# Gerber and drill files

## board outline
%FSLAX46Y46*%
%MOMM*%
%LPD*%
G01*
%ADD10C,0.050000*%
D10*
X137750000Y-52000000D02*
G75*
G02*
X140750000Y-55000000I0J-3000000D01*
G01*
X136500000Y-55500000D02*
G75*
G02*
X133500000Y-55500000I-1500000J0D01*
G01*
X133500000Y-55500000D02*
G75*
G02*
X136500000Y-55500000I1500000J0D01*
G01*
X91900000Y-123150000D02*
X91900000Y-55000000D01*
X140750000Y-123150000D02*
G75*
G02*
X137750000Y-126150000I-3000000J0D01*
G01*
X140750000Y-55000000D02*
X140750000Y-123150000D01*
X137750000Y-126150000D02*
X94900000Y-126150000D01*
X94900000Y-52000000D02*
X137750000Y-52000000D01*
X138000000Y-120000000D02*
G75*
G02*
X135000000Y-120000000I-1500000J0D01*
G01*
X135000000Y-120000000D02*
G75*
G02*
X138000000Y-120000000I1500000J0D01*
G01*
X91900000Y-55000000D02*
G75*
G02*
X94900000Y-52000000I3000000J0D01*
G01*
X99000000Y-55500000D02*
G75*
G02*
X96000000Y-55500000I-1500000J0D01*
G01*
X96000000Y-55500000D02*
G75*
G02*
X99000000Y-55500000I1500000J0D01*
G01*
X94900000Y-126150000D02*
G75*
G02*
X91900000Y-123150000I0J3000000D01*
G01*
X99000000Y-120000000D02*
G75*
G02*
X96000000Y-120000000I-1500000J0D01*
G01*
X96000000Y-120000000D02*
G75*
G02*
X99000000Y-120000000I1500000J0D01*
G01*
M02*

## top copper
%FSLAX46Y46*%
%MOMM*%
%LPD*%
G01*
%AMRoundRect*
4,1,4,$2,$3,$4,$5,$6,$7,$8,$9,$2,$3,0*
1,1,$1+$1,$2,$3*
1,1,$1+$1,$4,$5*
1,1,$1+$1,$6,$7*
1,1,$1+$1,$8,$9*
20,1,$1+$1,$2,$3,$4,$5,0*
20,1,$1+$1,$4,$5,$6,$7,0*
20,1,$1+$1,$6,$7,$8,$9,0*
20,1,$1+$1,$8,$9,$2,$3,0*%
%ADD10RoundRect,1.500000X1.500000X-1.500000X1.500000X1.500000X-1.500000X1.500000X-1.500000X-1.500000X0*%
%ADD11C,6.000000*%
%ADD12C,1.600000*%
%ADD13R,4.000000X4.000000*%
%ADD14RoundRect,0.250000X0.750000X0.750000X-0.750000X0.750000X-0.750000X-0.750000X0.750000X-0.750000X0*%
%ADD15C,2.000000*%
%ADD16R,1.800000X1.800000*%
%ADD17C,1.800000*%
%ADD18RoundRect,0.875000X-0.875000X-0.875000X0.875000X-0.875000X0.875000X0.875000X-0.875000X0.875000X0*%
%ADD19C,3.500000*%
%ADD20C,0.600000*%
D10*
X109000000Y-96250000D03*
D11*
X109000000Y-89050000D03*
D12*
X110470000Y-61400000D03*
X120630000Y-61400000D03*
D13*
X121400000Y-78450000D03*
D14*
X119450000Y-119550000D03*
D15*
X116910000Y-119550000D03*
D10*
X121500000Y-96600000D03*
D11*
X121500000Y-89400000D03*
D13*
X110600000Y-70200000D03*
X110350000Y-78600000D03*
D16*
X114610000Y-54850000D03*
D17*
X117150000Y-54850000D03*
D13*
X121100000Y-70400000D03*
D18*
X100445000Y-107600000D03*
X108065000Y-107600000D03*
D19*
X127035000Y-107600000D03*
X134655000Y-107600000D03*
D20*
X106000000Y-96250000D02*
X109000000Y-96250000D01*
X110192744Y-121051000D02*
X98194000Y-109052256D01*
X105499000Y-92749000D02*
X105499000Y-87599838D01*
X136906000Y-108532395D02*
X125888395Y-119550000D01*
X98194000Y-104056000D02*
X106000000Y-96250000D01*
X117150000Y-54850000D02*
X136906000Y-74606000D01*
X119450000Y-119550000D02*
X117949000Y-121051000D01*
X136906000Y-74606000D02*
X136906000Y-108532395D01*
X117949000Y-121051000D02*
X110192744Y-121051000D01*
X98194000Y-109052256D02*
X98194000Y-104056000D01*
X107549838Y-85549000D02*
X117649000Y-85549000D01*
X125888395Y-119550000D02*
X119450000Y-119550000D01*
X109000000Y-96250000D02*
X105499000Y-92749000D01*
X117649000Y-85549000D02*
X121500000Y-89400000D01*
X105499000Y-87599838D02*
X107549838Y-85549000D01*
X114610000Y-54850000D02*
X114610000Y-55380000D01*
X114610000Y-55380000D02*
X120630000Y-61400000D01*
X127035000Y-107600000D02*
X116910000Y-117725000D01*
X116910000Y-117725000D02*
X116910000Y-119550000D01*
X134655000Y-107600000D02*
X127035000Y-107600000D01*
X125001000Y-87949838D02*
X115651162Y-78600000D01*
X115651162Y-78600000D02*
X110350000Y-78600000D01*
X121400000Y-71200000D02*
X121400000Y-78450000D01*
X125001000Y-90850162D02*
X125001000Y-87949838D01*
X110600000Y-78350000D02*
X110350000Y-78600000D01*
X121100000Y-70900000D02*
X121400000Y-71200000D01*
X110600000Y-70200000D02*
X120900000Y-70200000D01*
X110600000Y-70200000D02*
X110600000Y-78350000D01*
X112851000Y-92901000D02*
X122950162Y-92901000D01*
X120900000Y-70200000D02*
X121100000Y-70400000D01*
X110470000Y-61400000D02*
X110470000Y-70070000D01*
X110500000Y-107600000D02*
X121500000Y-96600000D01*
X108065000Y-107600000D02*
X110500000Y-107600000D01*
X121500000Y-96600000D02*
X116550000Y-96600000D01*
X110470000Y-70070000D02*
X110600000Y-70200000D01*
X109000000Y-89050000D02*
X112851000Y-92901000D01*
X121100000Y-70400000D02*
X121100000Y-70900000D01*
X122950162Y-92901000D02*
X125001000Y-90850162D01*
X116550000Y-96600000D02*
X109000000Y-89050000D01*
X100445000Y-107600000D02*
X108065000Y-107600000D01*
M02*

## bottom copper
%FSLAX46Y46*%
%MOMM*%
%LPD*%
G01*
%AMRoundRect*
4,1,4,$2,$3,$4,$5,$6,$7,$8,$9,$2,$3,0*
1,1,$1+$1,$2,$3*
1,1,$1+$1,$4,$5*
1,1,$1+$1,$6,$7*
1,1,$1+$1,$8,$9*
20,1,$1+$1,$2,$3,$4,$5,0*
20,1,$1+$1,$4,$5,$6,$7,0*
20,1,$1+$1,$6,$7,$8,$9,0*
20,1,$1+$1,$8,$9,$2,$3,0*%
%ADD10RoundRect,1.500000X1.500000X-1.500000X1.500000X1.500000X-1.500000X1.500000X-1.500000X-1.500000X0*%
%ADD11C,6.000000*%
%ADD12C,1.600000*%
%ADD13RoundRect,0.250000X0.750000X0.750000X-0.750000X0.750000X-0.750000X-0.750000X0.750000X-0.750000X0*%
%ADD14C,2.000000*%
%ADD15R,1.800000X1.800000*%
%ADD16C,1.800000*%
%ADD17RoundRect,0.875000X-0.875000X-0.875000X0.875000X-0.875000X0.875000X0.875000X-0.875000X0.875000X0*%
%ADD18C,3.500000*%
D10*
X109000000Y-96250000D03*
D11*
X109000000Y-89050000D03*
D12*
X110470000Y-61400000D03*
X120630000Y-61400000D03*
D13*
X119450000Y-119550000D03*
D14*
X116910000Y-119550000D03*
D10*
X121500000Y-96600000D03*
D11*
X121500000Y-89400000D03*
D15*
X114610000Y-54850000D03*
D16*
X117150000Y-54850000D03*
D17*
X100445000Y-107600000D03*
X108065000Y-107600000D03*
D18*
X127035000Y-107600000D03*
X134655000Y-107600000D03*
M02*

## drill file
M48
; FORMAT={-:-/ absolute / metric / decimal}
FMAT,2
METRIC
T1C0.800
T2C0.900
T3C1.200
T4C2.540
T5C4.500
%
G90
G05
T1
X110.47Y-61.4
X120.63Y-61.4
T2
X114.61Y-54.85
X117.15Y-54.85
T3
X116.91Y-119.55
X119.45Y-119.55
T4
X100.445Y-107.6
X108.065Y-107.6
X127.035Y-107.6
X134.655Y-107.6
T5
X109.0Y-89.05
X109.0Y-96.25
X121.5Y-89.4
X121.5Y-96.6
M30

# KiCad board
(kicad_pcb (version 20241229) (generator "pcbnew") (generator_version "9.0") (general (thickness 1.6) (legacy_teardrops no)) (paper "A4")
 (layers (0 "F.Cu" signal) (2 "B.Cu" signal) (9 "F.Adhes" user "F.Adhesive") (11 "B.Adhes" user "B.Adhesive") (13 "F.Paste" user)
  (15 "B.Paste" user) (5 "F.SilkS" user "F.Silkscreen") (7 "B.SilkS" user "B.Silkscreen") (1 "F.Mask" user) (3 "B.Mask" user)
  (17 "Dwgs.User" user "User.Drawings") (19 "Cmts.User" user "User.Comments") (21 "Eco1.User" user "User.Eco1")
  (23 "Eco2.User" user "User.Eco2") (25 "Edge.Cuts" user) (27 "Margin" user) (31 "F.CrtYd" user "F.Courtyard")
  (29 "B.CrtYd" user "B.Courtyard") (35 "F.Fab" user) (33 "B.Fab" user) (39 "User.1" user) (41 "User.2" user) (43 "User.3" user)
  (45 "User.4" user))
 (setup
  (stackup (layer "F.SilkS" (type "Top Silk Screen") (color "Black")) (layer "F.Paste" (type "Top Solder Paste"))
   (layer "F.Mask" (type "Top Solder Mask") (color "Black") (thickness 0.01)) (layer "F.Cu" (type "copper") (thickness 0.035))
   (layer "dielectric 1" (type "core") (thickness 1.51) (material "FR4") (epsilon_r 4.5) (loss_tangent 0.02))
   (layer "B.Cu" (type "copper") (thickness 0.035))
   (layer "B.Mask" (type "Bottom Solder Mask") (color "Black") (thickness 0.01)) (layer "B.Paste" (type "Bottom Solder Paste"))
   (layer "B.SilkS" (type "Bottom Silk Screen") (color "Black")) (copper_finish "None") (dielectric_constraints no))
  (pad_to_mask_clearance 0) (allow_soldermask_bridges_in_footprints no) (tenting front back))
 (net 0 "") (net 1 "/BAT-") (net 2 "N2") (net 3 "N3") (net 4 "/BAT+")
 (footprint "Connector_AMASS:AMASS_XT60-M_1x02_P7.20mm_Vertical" (layer "F.Cu") (at 109 96.25 90)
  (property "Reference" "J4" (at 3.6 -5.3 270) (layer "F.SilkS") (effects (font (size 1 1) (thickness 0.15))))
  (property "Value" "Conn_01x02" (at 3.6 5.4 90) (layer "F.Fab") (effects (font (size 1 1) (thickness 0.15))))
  (pad "1" thru_hole roundrect (at 0 0 90) (size 6 6) (drill 4.5) (layers "*.Cu" "*.Mask") (remove_unused_layers no) (roundrect_rratio 0.25)
   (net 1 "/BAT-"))
  (pad "2" thru_hole circle (at 7.2 0 90) (size 6 6) (drill 4.5) (layers "*.Cu" "*.Mask") (remove_unused_layers no) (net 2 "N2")))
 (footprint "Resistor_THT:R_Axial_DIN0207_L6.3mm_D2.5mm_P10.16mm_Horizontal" (layer "F.Cu") (at 110.47 61.4)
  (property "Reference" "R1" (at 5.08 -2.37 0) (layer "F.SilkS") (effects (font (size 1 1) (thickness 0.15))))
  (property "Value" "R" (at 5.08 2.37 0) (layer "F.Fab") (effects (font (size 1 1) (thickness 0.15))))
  (pad "1" thru_hole circle (at 0 0) (size 1.6 1.6) (drill 0.8) (layers "*.Cu" "*.Mask") (remove_unused_layers no) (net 2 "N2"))
  (pad "2" thru_hole circle (at 10.16 0) (size 1.6 1.6) (drill 0.8) (layers "*.Cu" "*.Mask") (remove_unused_layers no) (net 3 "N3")))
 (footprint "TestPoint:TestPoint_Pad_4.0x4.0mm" (layer "F.Cu") (at 121.4 78.45)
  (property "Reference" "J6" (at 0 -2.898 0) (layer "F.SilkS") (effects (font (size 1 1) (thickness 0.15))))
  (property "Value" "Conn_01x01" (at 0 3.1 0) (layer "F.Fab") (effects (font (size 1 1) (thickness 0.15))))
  (pad "1" smd rect (at 0 0) (size 4 4) (layers "F.Cu" "F.Mask") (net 2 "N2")))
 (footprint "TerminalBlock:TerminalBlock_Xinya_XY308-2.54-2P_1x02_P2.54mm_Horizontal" (layer "F.Cu") (at 119.45 119.55 180)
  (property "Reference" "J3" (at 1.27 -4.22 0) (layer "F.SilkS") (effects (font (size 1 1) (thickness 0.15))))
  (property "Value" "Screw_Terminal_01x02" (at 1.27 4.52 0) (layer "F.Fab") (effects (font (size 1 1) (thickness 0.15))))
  (pad "1" thru_hole roundrect (at 0 0 180) (size 2 2) (drill 1.2) (layers "*.Cu" "*.Mask") (remove_unused_layers no)
   (roundrect_rratio 0.125) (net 1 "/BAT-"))
  (pad "2" thru_hole circle (at 2.54 0 180) (size 2 2) (drill 1.2) (layers "*.Cu" "*.Mask") (remove_unused_layers no) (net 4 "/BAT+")))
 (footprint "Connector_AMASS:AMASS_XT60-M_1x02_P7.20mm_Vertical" (layer "F.Cu") (at 121.5 96.6 90)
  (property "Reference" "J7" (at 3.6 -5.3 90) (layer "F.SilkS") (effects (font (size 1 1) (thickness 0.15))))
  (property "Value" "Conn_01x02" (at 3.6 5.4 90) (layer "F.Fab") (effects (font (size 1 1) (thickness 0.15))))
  (pad "1" thru_hole roundrect (at 0 0 90) (size 6 6) (drill 4.5) (layers "*.Cu" "*.Mask") (remove_unused_layers no) (roundrect_rratio 0.25)
   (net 2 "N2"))
  (pad "2" thru_hole circle (at 7.2 0 90) (size 6 6) (drill 4.5) (layers "*.Cu" "*.Mask") (remove_unused_layers no) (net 1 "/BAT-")))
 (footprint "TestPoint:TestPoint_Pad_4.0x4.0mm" (layer "F.Cu") (at 110.6 70.2)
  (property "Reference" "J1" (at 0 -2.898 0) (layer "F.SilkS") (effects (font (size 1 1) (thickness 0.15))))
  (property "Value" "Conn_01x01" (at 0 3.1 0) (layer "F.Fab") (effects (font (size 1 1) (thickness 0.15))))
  (pad "1" smd rect (at 0 0) (size 4 4) (layers "F.Cu" "F.Mask") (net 2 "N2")))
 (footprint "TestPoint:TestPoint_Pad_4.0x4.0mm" (layer "F.Cu") (at 110.35 78.6)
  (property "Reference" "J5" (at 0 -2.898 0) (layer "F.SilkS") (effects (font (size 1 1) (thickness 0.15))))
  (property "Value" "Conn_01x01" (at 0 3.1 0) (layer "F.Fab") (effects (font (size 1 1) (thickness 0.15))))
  (pad "1" smd rect (at 0 0) (size 4 4) (layers "F.Cu" "F.Mask") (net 2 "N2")))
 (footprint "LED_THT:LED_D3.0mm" (layer "F.Cu") (at 114.61 54.85)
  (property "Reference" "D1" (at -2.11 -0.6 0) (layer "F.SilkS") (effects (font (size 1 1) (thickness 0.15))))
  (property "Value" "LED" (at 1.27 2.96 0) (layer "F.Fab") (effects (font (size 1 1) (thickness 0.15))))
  (pad "1" thru_hole rect (at 0 0) (size 1.8 1.8) (drill 0.9) (layers "*.Cu" "*.Mask") (remove_unused_layers no) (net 3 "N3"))
  (pad "2" thru_hole circle (at 2.54 0) (size 1.8 1.8) (drill 0.9) (layers "*.Cu" "*.Mask") (remove_unused_layers no) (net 1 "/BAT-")))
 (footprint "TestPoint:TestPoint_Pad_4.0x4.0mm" (layer "F.Cu") (at 121.1 70.4)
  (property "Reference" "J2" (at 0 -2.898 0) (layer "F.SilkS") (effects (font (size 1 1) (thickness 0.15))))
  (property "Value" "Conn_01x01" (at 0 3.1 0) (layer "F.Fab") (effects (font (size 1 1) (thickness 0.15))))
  (pad "1" smd rect (at 0 0) (size 4 4) (layers "F.Cu" "F.Mask") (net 2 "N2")))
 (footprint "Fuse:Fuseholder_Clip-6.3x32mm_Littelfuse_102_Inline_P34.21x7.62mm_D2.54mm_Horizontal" (layer "B.Cu") (at 100.445 107.6)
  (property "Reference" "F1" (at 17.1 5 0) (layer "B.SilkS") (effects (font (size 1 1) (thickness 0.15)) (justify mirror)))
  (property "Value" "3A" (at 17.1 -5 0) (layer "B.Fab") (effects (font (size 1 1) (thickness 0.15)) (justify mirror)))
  (pad "1" thru_hole roundrect (at 0 0) (size 3.5 3.5) (drill 2.54) (layers "*.Cu" "*.Mask") (remove_unused_layers no)
   (roundrect_rratio 0.25) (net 2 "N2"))
  (pad "1" thru_hole roundrect (at 7.62 0) (size 3.5 3.5) (drill 2.54) (layers "*.Cu" "*.Mask") (remove_unused_layers no)
   (roundrect_rratio 0.25) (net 2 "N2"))
  (pad "2" thru_hole circle (at 26.59 0) (size 3.5 3.5) (drill 2.54) (layers "*.Cu" "*.Mask") (remove_unused_layers no) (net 4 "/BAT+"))
  (pad "2" thru_hole circle (at 34.21 0) (size 3.5 3.5) (drill 2.54) (layers "*.Cu" "*.Mask") (remove_unused_layers no) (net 4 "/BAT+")))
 (gr_arc (start 137.75 52) (mid 139.87132 52.87868) (end 140.75 55) (stroke (width 0.05) (type default)) (layer "Edge.Cuts"))
 (gr_circle (center 135 55.5) (end 135 54) (stroke (width 0.05) (type default)) (fill no) (layer "Edge.Cuts"))
 (gr_line (start 91.9 123.15) (end 91.9 55) (stroke (width 0.05) (type default)) (layer "Edge.Cuts"))
 (gr_arc (start 140.75 123.15) (mid 139.87132 125.27132) (end 137.75 126.15) (stroke (width 0.05) (type default)) (layer "Edge.Cuts"))
 (gr_line (start 140.75 55) (end 140.75 123.15) (stroke (width 0.05) (type default)) (layer "Edge.Cuts"))
 (gr_line (start 137.75 126.15) (end 94.9 126.15) (stroke (width 0.05) (type default)) (layer "Edge.Cuts"))
 (gr_line (start 94.9 52) (end 137.75 52) (stroke (width 0.05) (type default)) (layer "Edge.Cuts"))
 (gr_circle (center 136.5 120) (end 136.5 121.5) (stroke (width 0.05) (type default)) (fill no) (layer "Edge.Cuts"))
 (gr_arc (start 91.9 55) (mid 92.77868 52.87868) (end 94.9 52) (stroke (width 0.05) (type default)) (layer "Edge.Cuts"))
 (gr_circle (center 97.5 55.5) (end 97.5 57) (stroke (width 0.05) (type default)) (fill no) (layer "Edge.Cuts"))
 (gr_arc (start 94.9 126.15) (mid 92.77868 125.27132) (end 91.9 123.15) (stroke (width 0.05) (type default)) (layer "Edge.Cuts"))
 (gr_circle (center 97.5 120) (end 97.5 121.5) (stroke (width 0.05) (type default)) (fill no) (layer "Edge.Cuts"))
 (segment (start 106 96.25) (end 109 96.25) (width 0.6) (layer "F.Cu") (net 1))
 (segment (start 110.192744 121.051) (end 98.194 109.052256) (width 0.6) (layer "F.Cu") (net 1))
 (segment (start 105.499 92.749) (end 105.499 87.599838) (width 0.6) (layer "F.Cu") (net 1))
 (segment (start 136.906 108.532395) (end 125.888395 119.55) (width 0.6) (layer "F.Cu") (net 1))
 (segment (start 98.194 104.056) (end 106 96.25) (width 0.6) (layer "F.Cu") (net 1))
 (segment (start 117.15 54.85) (end 136.906 74.606) (width 0.6) (layer "F.Cu") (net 1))
 (segment (start 119.45 119.55) (end 117.949 121.051) (width 0.6) (layer "F.Cu") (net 1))
 (segment (start 136.906 74.606) (end 136.906 108.532395) (width 0.6) (layer "F.Cu") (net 1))
 (segment (start 117.949 121.051) (end 110.192744 121.051) (width 0.6) (layer "F.Cu") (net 1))
 (segment (start 98.194 109.052256) (end 98.194 104.056) (width 0.6) (layer "F.Cu") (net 1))
 (segment (start 107.549838 85.549) (end 117.649 85.549) (width 0.6) (layer "F.Cu") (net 1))
 (segment (start 125.888395 119.55) (end 119.45 119.55) (width 0.6) (layer "F.Cu") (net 1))
 (segment (start 109 96.25) (end 105.499 92.749) (width 0.6) (layer "F.Cu") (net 1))
 (segment (start 117.649 85.549) (end 121.5 89.4) (width 0.6) (layer "F.Cu") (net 1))
 (segment (start 105.499 87.599838) (end 107.549838 85.549) (width 0.6) (layer "F.Cu") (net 1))
 (segment (start 114.61 54.85) (end 114.61 55.38) (width 0.6) (layer "F.Cu") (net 3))
 (segment (start 114.61 55.38) (end 120.63 61.4) (width 0.6) (layer "F.Cu") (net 3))
 (segment (start 127.035 107.6) (end 116.91 117.725) (width 0.6) (layer "F.Cu") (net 4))
 (segment (start 116.91 117.725) (end 116.91 119.55) (width 0.6) (layer "F.Cu") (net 4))
 (segment (start 134.655 107.6) (end 127.035 107.6) (width 0.6) (layer "F.Cu") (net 4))
 (segment (start 125.001 87.949838) (end 115.651162 78.6) (width 0.6) (layer "F.Cu") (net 2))
 (segment (start 115.651162 78.6) (end 110.35 78.6) (width 0.6) (layer "F.Cu") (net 2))
 (segment (start 121.4 71.2) (end 121.4 78.45) (width 0.6) (layer "F.Cu") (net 2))
 (segment (start 125.001 90.850162) (end 125.001 87.949838) (width 0.6) (layer "F.Cu") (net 2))
 (segment (start 110.6 78.35) (end 110.35 78.6) (width 0.6) (layer "F.Cu") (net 2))
 (segment (start 121.1 70.9) (end 121.4 71.2) (width 0.6) (layer "F.Cu") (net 2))
 (segment (start 110.6 70.2) (end 120.9 70.2) (width 0.6) (layer "F.Cu") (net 2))
 (segment (start 110.6 70.2) (end 110.6 78.35) (width 0.6) (layer "F.Cu") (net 2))
 (segment (start 112.851 92.901) (end 122.950162 92.901) (width 0.6) (layer "F.Cu") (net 2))
 (segment (start 120.9 70.2) (end 121.1 70.4) (width 0.6) (layer "F.Cu") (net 2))
 (segment (start 110.47 61.4) (end 110.47 70.07) (width 0.6) (layer "F.Cu") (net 2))
 (segment (start 110.5 107.6) (end 121.5 96.6) (width 0.6) (layer "F.Cu") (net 2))
 (segment (start 108.065 107.6) (end 110.5 107.6) (width 0.6) (layer "F.Cu") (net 2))
 (segment (start 121.5 96.6) (end 116.55 96.6) (width 0.6) (layer "F.Cu") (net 2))
 (segment (start 110.47 70.07) (end 110.6 70.2) (width 0.6) (layer "F.Cu") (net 2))
 (segment (start 109 89.05) (end 112.851 92.901) (width 0.6) (layer "F.Cu") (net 2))
 (segment (start 121.1 70.4) (end 121.1 70.9) (width 0.6) (layer "F.Cu") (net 2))
 (segment (start 122.950162 92.901) (end 125.001 90.850162) (width 0.6) (layer "F.Cu") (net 2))
 (segment (start 116.55 96.6) (end 109 89.05) (width 0.6) (layer "F.Cu") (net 2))
 (segment (start 100.445 107.6) (end 108.065 107.6) (width 0.6) (layer "F.Cu") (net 2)))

